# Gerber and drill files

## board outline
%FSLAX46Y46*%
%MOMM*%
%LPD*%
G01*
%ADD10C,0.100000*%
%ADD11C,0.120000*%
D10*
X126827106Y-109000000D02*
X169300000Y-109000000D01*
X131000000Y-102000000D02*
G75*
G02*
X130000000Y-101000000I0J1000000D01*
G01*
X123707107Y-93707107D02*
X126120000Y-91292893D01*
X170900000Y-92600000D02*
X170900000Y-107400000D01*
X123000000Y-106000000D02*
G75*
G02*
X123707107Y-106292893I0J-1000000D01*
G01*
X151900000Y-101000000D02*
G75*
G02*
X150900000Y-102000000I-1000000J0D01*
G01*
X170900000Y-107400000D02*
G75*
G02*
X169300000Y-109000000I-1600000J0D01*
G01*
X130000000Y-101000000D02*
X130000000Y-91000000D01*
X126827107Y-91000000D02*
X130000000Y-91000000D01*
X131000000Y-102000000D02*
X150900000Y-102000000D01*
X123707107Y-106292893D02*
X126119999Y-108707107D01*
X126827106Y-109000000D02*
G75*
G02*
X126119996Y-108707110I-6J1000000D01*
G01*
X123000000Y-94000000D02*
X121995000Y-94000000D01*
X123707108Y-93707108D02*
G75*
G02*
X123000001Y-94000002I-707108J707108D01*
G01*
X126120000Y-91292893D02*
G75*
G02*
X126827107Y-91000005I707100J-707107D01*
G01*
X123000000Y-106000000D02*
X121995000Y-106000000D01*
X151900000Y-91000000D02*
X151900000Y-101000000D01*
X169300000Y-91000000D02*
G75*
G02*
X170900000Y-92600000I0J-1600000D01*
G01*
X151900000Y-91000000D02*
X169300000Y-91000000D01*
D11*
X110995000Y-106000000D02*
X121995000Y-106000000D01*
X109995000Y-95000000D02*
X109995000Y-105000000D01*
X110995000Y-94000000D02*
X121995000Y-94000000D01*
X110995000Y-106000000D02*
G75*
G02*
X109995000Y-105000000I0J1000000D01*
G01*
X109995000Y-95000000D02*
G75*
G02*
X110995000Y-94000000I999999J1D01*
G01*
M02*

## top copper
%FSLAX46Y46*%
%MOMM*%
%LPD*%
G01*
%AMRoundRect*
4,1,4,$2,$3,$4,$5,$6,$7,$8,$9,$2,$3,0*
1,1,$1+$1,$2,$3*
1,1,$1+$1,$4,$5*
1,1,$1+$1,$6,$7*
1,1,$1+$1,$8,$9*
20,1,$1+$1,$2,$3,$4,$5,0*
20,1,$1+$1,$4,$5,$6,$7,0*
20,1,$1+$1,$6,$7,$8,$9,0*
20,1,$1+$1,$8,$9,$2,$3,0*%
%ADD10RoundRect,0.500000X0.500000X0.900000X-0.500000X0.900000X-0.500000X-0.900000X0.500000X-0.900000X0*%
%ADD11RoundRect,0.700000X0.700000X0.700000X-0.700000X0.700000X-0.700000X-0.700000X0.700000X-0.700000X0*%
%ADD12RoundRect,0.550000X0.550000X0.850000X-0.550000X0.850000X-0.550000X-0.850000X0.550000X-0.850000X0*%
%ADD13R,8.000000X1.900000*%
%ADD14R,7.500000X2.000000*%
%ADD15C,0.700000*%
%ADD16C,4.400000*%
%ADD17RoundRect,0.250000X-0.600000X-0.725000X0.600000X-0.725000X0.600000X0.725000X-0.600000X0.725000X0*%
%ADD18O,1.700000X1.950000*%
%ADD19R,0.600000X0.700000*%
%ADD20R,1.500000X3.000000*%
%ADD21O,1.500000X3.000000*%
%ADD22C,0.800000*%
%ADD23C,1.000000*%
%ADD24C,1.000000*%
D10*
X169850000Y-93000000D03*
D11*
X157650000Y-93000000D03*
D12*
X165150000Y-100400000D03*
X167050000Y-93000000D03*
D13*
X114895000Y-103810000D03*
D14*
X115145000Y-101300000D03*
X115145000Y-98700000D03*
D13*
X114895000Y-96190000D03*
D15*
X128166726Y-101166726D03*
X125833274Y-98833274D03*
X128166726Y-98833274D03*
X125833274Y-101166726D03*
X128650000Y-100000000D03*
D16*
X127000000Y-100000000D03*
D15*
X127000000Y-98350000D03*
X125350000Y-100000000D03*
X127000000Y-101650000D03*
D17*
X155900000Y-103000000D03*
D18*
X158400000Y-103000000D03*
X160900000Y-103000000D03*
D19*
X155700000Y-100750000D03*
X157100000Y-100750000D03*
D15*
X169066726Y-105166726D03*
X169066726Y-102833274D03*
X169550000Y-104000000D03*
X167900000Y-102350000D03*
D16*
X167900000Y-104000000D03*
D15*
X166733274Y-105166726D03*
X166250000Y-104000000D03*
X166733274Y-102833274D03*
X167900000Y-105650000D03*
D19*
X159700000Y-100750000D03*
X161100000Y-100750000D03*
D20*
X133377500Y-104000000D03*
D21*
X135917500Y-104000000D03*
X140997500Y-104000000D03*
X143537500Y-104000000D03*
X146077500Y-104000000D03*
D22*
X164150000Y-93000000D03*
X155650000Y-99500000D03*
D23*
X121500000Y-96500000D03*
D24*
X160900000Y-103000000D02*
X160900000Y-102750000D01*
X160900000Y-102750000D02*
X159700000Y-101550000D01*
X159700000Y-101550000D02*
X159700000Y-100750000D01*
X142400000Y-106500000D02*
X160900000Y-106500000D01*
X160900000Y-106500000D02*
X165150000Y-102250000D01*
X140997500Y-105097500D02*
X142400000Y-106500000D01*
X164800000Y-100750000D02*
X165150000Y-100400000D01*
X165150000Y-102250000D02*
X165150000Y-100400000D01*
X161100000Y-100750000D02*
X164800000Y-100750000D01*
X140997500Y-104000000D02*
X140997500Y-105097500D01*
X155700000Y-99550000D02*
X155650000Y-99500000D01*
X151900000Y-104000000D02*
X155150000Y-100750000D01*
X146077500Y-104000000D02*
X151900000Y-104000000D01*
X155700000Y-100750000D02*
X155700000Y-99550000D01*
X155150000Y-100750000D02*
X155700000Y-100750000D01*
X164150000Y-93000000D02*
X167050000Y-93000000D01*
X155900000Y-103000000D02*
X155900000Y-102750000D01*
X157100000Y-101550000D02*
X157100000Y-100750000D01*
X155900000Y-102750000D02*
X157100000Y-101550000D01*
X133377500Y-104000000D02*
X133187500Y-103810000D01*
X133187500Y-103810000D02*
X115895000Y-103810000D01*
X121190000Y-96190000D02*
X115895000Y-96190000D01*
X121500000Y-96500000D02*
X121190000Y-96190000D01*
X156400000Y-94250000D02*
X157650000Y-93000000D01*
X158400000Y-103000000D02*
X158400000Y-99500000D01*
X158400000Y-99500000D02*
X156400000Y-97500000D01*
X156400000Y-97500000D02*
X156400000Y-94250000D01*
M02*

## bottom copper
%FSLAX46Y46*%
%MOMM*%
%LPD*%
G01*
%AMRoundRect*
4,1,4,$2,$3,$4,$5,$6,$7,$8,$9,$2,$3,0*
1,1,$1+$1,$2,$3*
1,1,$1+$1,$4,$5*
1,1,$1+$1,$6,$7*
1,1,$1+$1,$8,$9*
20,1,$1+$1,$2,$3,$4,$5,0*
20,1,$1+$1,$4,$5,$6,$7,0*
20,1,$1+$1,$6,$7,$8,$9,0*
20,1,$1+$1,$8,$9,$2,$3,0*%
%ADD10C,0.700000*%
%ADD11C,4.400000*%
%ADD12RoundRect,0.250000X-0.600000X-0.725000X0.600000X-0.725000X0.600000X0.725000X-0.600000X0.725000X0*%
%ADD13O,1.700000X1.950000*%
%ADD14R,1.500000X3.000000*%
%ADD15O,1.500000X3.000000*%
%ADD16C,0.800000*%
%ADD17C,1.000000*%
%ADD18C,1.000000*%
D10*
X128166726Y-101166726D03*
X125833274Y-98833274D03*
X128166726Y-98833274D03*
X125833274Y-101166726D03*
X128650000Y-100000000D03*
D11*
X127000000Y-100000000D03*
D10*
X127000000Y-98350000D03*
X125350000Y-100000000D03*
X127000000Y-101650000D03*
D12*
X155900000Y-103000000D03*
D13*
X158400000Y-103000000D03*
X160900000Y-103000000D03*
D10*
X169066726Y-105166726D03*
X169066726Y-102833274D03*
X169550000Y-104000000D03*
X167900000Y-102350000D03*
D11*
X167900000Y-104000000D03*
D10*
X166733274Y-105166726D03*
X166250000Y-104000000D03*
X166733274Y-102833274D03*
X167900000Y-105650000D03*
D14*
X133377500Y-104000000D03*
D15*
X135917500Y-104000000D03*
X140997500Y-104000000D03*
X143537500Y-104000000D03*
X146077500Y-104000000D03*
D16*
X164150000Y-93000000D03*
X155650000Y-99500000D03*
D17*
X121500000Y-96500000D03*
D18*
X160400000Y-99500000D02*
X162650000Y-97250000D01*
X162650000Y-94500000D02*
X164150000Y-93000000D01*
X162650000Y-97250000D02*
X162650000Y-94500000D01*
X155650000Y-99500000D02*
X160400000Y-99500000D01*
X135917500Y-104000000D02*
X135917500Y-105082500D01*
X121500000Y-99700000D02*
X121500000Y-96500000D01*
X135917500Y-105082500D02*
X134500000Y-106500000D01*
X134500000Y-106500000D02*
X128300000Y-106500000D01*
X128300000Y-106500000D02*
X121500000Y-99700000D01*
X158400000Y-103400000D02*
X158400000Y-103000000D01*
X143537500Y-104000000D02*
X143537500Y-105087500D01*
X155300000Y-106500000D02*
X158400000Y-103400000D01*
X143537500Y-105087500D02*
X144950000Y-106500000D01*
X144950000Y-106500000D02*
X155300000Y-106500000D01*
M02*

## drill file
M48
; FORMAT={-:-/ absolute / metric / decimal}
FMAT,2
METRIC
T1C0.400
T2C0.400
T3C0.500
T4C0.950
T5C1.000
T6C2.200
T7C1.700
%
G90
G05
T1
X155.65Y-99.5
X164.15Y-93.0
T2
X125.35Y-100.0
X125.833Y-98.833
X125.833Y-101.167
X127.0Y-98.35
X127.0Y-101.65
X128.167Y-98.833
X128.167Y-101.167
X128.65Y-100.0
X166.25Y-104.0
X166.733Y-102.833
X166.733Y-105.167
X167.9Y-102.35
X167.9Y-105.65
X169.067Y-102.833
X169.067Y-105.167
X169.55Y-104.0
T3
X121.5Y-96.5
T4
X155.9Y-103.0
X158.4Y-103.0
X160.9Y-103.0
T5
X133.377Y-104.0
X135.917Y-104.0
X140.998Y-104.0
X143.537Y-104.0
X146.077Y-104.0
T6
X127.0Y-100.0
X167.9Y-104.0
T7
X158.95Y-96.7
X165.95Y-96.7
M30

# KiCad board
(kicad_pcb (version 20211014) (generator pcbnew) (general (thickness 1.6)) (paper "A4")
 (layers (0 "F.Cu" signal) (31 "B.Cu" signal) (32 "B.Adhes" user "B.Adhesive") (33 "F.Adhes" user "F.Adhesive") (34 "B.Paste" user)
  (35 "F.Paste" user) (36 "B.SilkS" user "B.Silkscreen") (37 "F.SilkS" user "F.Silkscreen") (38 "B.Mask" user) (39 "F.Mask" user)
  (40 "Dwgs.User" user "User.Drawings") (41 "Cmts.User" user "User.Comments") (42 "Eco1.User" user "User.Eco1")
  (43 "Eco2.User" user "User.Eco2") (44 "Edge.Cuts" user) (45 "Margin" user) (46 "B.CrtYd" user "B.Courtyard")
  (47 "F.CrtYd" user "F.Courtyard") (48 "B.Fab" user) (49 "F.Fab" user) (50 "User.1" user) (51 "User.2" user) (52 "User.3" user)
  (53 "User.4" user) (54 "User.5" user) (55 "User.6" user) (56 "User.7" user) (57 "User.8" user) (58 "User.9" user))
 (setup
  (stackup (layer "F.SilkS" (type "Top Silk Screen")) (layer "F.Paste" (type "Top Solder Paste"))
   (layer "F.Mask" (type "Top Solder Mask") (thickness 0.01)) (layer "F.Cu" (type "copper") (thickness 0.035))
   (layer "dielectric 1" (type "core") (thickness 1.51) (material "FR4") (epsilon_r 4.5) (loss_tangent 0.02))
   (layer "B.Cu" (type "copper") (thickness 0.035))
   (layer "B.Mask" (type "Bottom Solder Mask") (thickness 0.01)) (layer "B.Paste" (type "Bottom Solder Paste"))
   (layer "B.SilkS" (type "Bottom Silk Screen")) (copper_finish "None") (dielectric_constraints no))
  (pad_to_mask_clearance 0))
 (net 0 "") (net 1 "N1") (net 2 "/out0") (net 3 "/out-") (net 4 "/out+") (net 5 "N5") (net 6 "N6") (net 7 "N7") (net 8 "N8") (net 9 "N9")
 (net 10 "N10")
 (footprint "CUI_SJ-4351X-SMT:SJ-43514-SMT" (layer "F.Cu") (at 170.45 96.7 180)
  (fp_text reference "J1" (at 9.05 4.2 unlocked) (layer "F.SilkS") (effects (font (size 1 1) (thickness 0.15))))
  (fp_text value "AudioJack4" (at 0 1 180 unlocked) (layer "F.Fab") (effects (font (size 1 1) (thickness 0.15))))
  (pad "" np_thru_hole circle (at 11.5 0 180) (size 1.7 1.7) (drill 1.7) (layers *.Mask))
  (pad "" np_thru_hole circle (at 4.5 0 180) (size 1.7 1.7) (drill 1.7) (layers *.Mask))
  (pad "1" smd roundrect (at 0.6 3.7 180) (size 2 2.8) (layers "F.Cu" "F.Paste" "F.Mask") (roundrect_rratio 0.25) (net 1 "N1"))
  (pad "2" smd roundrect (at 12.8 3.7 180) (size 2.8 2.8) (layers "F.Cu" "F.Paste" "F.Mask") (roundrect_rratio 0.25) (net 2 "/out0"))
  (pad "3" smd roundrect (at 5.3 -3.7 180) (size 2.2 2.8) (layers "F.Cu" "F.Paste" "F.Mask") (roundrect_rratio 0.25) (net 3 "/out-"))
  (pad "4" smd roundrect (at 3.4 3.7 180) (size 2.2 2.8) (layers "F.Cu" "F.Paste" "F.Mask") (roundrect_rratio 0.25) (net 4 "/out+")))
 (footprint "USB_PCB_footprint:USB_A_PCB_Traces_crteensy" (layer "F.Cu") (at 109.995 100 -90)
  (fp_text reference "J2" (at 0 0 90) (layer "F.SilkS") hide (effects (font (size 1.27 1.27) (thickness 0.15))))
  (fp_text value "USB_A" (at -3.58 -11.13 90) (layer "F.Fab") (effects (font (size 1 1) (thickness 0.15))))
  (fp_line (start 6 -1) (end 6 -12) (layer "Edge.Cuts") (width 0.12))
  (fp_line (start -5 0) (end 5 0) (layer "Edge.Cuts") (width 0.12))
  (fp_line (start -6 -1) (end -6 -12) (layer "Edge.Cuts") (width 0.12))
  (fp_arc (start 6 -1) (mid 5.707107 -0.292893) (end 5 0) (layer "Edge.Cuts") (width 0.12))
  (fp_arc (start -5 0) (mid -5.707107 -0.292893) (end -6 -1) (layer "Edge.Cuts") (width 0.12))
  (pad "1" connect rect (at 3.81 -4.9 270) (size 1.9 8) (layers "F.Cu" "F.Mask") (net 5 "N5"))
  (pad "2" connect rect (at 1.3 -5.15 270) (size 2 7.5) (layers "F.Cu" "F.Mask") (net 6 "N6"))
  (pad "3" connect rect (at -1.3 -5.15 270) (size 2 7.5) (layers "F.Cu" "F.Mask") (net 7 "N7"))
  (pad "4" connect rect (at -3.81 -4.9 270) (size 1.9 8) (layers "F.Cu" "F.Mask") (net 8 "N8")))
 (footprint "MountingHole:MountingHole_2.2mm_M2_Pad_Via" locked (layer "F.Cu") (at 127 100)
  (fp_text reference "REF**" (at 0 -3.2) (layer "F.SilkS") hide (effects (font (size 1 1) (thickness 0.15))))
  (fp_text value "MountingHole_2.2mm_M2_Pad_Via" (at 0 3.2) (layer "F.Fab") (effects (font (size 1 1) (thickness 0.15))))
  (pad "1" thru_hole circle locked (at 1.166726 1.166726) (size 0.7 0.7) (drill 0.4) (layers *.Cu *.Mask))
  (pad "1" thru_hole circle locked (at -1.166726 -1.166726) (size 0.7 0.7) (drill 0.4) (layers *.Cu *.Mask))
  (pad "1" thru_hole circle locked (at 1.166726 -1.166726) (size 0.7 0.7) (drill 0.4) (layers *.Cu *.Mask))
  (pad "1" thru_hole circle locked (at -1.166726 1.166726) (size 0.7 0.7) (drill 0.4) (layers *.Cu *.Mask))
  (pad "1" thru_hole circle locked (at 1.65 0) (size 0.7 0.7) (drill 0.4) (layers *.Cu *.Mask))
  (pad "1" thru_hole circle locked (at 0 0) (size 4.4 4.4) (drill 2.2) (layers *.Cu *.Mask))
  (pad "1" thru_hole circle locked (at 0 -1.65) (size 0.7 0.7) (drill 0.4) (layers *.Cu *.Mask))
  (pad "1" thru_hole circle locked (at -1.65 0) (size 0.7 0.7) (drill 0.4) (layers *.Cu *.Mask))
  (pad "1" thru_hole circle locked (at 0 1.65) (size 0.7 0.7) (drill 0.4) (layers *.Cu *.Mask)))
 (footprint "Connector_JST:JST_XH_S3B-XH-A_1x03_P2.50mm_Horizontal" (layer "F.Cu") (at 155.9 103)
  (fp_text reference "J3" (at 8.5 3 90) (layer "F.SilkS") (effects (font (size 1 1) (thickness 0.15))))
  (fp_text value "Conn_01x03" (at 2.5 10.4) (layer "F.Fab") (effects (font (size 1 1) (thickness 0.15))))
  (pad "1" thru_hole roundrect (at 0 0) (size 1.7 1.95) (drill 0.95) (layers *.Cu *.Mask) (roundrect_rratio 0.1470588235) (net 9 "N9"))
  (pad "2" thru_hole oval (at 2.5 0) (size 1.7 1.95) (drill 0.95) (layers *.Cu *.Mask) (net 2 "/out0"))
  (pad "3" thru_hole oval (at 5 0) (size 1.7 1.95) (drill 0.95) (layers *.Cu *.Mask) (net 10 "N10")))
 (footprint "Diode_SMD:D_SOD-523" (layer "F.Cu") (at 156.4 100.75)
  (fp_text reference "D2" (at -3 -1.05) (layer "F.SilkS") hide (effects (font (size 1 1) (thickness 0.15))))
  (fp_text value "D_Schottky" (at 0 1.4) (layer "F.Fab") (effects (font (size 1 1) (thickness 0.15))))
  (pad "1" smd rect (at -0.7 0 180) (size 0.6 0.7) (layers "F.Cu" "F.Paste" "F.Mask") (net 4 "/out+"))
  (pad "2" smd rect (at 0.7 0 180) (size 0.6 0.7) (layers "F.Cu" "F.Paste" "F.Mask") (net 9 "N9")))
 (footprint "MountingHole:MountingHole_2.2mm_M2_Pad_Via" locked (layer "F.Cu") (at 167.9 104)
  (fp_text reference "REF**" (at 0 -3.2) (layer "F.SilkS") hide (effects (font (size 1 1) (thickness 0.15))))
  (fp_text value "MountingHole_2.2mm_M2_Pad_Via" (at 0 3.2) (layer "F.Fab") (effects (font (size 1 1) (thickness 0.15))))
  (pad "1" thru_hole circle locked (at 1.166726 1.166726) (size 0.7 0.7) (drill 0.4) (layers *.Cu *.Mask))
  (pad "1" thru_hole circle locked (at 1.166726 -1.166726) (size 0.7 0.7) (drill 0.4) (layers *.Cu *.Mask))
  (pad "1" thru_hole circle locked (at 1.65 0) (size 0.7 0.7) (drill 0.4) (layers *.Cu *.Mask))
  (pad "1" thru_hole circle locked (at 0 -1.65) (size 0.7 0.7) (drill 0.4) (layers *.Cu *.Mask))
  (pad "1" thru_hole circle locked (at 0 0) (size 4.4 4.4) (drill 2.2) (layers *.Cu *.Mask))
  (pad "1" thru_hole circle locked (at -1.166726 1.166726) (size 0.7 0.7) (drill 0.4) (layers *.Cu *.Mask))
  (pad "1" thru_hole circle locked (at -1.65 0) (size 0.7 0.7) (drill 0.4) (layers *.Cu *.Mask))
  (pad "1" thru_hole circle locked (at -1.166726 -1.166726) (size 0.7 0.7) (drill 0.4) (layers *.Cu *.Mask))
  (pad "1" thru_hole circle locked (at 0 1.65) (size 0.7 0.7) (drill 0.4) (layers *.Cu *.Mask)))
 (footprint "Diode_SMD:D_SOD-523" (layer "F.Cu") (at 160.4 100.75)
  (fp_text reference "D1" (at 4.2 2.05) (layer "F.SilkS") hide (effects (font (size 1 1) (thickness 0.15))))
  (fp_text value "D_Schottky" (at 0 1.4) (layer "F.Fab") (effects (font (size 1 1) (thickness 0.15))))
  (pad "1" smd rect (at -0.7 0 180) (size 0.6 0.7) (layers "F.Cu" "F.Paste" "F.Mask") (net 10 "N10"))
  (pad "2" smd rect (at 0.7 0 180) (size 0.6 0.7) (layers "F.Cu" "F.Paste" "F.Mask") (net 3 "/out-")))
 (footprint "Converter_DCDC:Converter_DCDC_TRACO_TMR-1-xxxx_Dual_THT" (layer "B.Cu") (at 133.3775 104)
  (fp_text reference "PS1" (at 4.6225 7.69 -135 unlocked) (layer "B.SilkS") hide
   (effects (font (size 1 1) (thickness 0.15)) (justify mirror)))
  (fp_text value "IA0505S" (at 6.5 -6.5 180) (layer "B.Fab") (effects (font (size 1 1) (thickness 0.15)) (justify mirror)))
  (pad "1" thru_hole rect (at 0 0) (size 1.5 3) (drill 1) (layers *.Cu *.Mask) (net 5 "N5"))
  (pad "2" thru_hole oval (at 2.54 0) (size 1.5 3) (drill 1) (layers *.Cu *.Mask) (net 8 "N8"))
  (pad "4" thru_hole oval (at 7.62 0) (size 1.5 3) (drill 1) (layers *.Cu *.Mask) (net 3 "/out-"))
  (pad "5" thru_hole oval (at 10.16 0) (size 1.5 3) (drill 1) (layers *.Cu *.Mask) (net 2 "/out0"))
  (pad "6" thru_hole oval (at 12.7 0) (size 1.5 3) (drill 1) (layers *.Cu *.Mask) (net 4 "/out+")))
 (gr_line (start 126.827106 109) (end 169.3 109) (layer "Edge.Cuts") (width 0.1))
 (gr_arc (start 131 102) (mid 130.292893 101.707107) (end 130 101) (layer "Edge.Cuts") (width 0.1))
 (gr_line (start 123.707107 93.707107) (end 126.12 91.292893) (layer "Edge.Cuts") (width 0.1))
 (gr_line (start 170.9 92.6) (end 170.9 107.4) (layer "Edge.Cuts") (width 0.1))
 (gr_arc (start 123 106) (mid 123.382683 106.07612) (end 123.707107 106.292893) (layer "Edge.Cuts") (width 0.1))
 (gr_arc (start 151.9 101) (mid 151.607107 101.707107) (end 150.9 102) (layer "Edge.Cuts") (width 0.1))
 (gr_arc (start 170.9 107.4) (mid 170.431371 108.531371) (end 169.3 109) (layer "Edge.Cuts") (width 0.1))
 (gr_line (start 130 101) (end 130 91) (layer "Edge.Cuts") (width 0.1))
 (gr_line (start 126.827107 91) (end 130 91) (layer "Edge.Cuts") (width 0.1))
 (gr_line (start 131 102) (end 150.9 102) (layer "Edge.Cuts") (width 0.1))
 (gr_line (start 123.707107 106.292893) (end 126.119999 108.707107) (layer "Edge.Cuts") (width 0.1))
 (gr_arc (start 126.827106 109) (mid 126.444423 108.92388) (end 126.119999 108.707107) (layer "Edge.Cuts") (width 0.1))
 (gr_line (start 123 94) (end 121.995 94) (layer "Edge.Cuts") (width 0.1))
 (gr_arc (start 123.707108 93.707108) (mid 123.382685 93.923881) (end 123.000001 94.000001) (layer "Edge.Cuts") (width 0.1))
 (gr_arc (start 126.12 91.292893) (mid 126.444423 91.07612) (end 126.827107 91) (layer "Edge.Cuts") (width 0.1))
 (gr_line (start 123 106) (end 121.995 106) (layer "Edge.Cuts") (width 0.1))
 (gr_line (start 151.9 91) (end 151.9 101) (layer "Edge.Cuts") (width 0.1))
 (gr_arc (start 169.3 91) (mid 170.431371 91.468629) (end 170.9 92.6) (layer "Edge.Cuts") (width 0.1))
 (gr_line (start 151.9 91) (end 169.3 91) (layer "Edge.Cuts") (width 0.1))
 (segment (start 160.9 103) (end 160.9 102.75) (width 1) (layer "F.Cu") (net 10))
 (segment (start 160.9 102.75) (end 159.7 101.55) (width 1) (layer "F.Cu") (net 10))
 (segment (start 159.7 101.55) (end 159.7 100.75) (width 1) (layer "F.Cu") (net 10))
 (segment (start 142.4 106.5) (end 160.9 106.5) (width 1) (layer "F.Cu") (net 3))
 (segment (start 160.9 106.5) (end 165.15 102.25) (width 1) (layer "F.Cu") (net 3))
 (segment (start 140.9975 105.0975) (end 142.4 106.5) (width 1) (layer "F.Cu") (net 3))
 (segment (start 164.8 100.75) (end 165.15 100.4) (width 1) (layer "F.Cu") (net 3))
 (segment (start 165.15 102.25) (end 165.15 100.4) (width 1) (layer "F.Cu") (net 3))
 (segment (start 161.1 100.75) (end 164.8 100.75) (width 1) (layer "F.Cu") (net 3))
 (segment (start 140.9975 104) (end 140.9975 105.0975) (width 1) (layer "F.Cu") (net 3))
 (segment (start 155.7 99.55) (end 155.65 99.5) (width 1) (layer "F.Cu") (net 4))
 (segment (start 151.9 104) (end 155.15 100.75) (width 1) (layer "F.Cu") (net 4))
 (segment (start 146.0775 104) (end 151.9 104) (width 1) (layer "F.Cu") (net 4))
 (segment (start 155.7 100.75) (end 155.7 99.55) (width 1) (layer "F.Cu") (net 4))
 (segment (start 155.15 100.75) (end 155.7 100.75) (width 1) (layer "F.Cu") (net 4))
 (segment (start 164.15 93) (end 167.05 93) (width 1) (layer "F.Cu") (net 4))
 (via (at 164.15 93) (size 0.8) (drill 0.4) (layers "F.Cu" "B.Cu") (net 4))
 (via (at 155.65 99.5) (size 0.8) (drill 0.4) (layers "F.Cu" "B.Cu") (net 4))
 (segment (start 160.4 99.5) (end 162.65 97.25) (width 1) (layer "B.Cu") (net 4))
 (segment (start 162.65 94.5) (end 164.15 93) (width 1) (layer "B.Cu") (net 4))
 (segment (start 162.65 97.25) (end 162.65 94.5) (width 1) (layer "B.Cu") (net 4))
 (segment (start 155.65 99.5) (end 160.4 99.5) (width 1) (layer "B.Cu") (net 4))
 (segment (start 155.9 103) (end 155.9 102.75) (width 1) (layer "F.Cu") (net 9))
 (segment (start 157.1 101.55) (end 157.1 100.75) (width 1) (layer "F.Cu") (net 9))
 (segment (start 155.9 102.75) (end 157.1 101.55) (width 1) (layer "F.Cu") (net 9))
 (segment (start 133.3775 104) (end 133.1875 103.81) (width 1) (layer "F.Cu") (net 5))
 (segment (start 133.1875 103.81) (end 115.895 103.81) (width 1) (layer "F.Cu") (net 5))
 (segment (start 121.19 96.19) (end 115.895 96.19) (width 1) (layer "F.Cu") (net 8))
 (segment (start 121.5 96.5) (end 121.19 96.19) (width 1) (layer "F.Cu") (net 8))
 (via (at 121.5 96.5) (size 1) (drill 0.5) (layers "F.Cu" "B.Cu") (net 8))
 (segment (start 135.9175 104) (end 135.9175 105.0825) (width 1) (layer "B.Cu") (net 8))
 (segment (start 121.5 99.7) (end 121.5 96.5) (width 1) (layer "B.Cu") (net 8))
 (segment (start 135.9175 105.0825) (end 134.5 106.5) (width 1) (layer "B.Cu") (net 8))
 (segment (start 134.5 106.5) (end 128.3 106.5) (width 1) (layer "B.Cu") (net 8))
 (segment (start 128.3 106.5) (end 121.5 99.7) (width 1) (layer "B.Cu") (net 8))
 (segment (start 156.4 94.25) (end 157.65 93) (width 1) (layer "F.Cu") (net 2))
 (segment (start 158.4 103) (end 158.4 99.5) (width 1) (layer "F.Cu") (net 2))
 (segment (start 158.4 99.5) (end 156.4 97.5) (width 1) (layer "F.Cu") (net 2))
 (segment (start 156.4 97.5) (end 156.4 94.25) (width 1) (layer "F.Cu") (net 2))
 (segment (start 158.4 103.4) (end 158.4 103) (width 1) (layer "B.Cu") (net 2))
 (segment (start 143.5375 104) (end 143.5375 105.0875) (width 1) (layer "B.Cu") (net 2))
 (segment (start 155.3 106.5) (end 158.4 103.4) (width 1) (layer "B.Cu") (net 2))
 (segment (start 143.5375 105.0875) (end 144.95 106.5) (width 1) (layer "B.Cu") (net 2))
 (segment (start 144.95 106.5) (end 155.3 106.5) (width 1) (layer "B.Cu") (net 2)))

